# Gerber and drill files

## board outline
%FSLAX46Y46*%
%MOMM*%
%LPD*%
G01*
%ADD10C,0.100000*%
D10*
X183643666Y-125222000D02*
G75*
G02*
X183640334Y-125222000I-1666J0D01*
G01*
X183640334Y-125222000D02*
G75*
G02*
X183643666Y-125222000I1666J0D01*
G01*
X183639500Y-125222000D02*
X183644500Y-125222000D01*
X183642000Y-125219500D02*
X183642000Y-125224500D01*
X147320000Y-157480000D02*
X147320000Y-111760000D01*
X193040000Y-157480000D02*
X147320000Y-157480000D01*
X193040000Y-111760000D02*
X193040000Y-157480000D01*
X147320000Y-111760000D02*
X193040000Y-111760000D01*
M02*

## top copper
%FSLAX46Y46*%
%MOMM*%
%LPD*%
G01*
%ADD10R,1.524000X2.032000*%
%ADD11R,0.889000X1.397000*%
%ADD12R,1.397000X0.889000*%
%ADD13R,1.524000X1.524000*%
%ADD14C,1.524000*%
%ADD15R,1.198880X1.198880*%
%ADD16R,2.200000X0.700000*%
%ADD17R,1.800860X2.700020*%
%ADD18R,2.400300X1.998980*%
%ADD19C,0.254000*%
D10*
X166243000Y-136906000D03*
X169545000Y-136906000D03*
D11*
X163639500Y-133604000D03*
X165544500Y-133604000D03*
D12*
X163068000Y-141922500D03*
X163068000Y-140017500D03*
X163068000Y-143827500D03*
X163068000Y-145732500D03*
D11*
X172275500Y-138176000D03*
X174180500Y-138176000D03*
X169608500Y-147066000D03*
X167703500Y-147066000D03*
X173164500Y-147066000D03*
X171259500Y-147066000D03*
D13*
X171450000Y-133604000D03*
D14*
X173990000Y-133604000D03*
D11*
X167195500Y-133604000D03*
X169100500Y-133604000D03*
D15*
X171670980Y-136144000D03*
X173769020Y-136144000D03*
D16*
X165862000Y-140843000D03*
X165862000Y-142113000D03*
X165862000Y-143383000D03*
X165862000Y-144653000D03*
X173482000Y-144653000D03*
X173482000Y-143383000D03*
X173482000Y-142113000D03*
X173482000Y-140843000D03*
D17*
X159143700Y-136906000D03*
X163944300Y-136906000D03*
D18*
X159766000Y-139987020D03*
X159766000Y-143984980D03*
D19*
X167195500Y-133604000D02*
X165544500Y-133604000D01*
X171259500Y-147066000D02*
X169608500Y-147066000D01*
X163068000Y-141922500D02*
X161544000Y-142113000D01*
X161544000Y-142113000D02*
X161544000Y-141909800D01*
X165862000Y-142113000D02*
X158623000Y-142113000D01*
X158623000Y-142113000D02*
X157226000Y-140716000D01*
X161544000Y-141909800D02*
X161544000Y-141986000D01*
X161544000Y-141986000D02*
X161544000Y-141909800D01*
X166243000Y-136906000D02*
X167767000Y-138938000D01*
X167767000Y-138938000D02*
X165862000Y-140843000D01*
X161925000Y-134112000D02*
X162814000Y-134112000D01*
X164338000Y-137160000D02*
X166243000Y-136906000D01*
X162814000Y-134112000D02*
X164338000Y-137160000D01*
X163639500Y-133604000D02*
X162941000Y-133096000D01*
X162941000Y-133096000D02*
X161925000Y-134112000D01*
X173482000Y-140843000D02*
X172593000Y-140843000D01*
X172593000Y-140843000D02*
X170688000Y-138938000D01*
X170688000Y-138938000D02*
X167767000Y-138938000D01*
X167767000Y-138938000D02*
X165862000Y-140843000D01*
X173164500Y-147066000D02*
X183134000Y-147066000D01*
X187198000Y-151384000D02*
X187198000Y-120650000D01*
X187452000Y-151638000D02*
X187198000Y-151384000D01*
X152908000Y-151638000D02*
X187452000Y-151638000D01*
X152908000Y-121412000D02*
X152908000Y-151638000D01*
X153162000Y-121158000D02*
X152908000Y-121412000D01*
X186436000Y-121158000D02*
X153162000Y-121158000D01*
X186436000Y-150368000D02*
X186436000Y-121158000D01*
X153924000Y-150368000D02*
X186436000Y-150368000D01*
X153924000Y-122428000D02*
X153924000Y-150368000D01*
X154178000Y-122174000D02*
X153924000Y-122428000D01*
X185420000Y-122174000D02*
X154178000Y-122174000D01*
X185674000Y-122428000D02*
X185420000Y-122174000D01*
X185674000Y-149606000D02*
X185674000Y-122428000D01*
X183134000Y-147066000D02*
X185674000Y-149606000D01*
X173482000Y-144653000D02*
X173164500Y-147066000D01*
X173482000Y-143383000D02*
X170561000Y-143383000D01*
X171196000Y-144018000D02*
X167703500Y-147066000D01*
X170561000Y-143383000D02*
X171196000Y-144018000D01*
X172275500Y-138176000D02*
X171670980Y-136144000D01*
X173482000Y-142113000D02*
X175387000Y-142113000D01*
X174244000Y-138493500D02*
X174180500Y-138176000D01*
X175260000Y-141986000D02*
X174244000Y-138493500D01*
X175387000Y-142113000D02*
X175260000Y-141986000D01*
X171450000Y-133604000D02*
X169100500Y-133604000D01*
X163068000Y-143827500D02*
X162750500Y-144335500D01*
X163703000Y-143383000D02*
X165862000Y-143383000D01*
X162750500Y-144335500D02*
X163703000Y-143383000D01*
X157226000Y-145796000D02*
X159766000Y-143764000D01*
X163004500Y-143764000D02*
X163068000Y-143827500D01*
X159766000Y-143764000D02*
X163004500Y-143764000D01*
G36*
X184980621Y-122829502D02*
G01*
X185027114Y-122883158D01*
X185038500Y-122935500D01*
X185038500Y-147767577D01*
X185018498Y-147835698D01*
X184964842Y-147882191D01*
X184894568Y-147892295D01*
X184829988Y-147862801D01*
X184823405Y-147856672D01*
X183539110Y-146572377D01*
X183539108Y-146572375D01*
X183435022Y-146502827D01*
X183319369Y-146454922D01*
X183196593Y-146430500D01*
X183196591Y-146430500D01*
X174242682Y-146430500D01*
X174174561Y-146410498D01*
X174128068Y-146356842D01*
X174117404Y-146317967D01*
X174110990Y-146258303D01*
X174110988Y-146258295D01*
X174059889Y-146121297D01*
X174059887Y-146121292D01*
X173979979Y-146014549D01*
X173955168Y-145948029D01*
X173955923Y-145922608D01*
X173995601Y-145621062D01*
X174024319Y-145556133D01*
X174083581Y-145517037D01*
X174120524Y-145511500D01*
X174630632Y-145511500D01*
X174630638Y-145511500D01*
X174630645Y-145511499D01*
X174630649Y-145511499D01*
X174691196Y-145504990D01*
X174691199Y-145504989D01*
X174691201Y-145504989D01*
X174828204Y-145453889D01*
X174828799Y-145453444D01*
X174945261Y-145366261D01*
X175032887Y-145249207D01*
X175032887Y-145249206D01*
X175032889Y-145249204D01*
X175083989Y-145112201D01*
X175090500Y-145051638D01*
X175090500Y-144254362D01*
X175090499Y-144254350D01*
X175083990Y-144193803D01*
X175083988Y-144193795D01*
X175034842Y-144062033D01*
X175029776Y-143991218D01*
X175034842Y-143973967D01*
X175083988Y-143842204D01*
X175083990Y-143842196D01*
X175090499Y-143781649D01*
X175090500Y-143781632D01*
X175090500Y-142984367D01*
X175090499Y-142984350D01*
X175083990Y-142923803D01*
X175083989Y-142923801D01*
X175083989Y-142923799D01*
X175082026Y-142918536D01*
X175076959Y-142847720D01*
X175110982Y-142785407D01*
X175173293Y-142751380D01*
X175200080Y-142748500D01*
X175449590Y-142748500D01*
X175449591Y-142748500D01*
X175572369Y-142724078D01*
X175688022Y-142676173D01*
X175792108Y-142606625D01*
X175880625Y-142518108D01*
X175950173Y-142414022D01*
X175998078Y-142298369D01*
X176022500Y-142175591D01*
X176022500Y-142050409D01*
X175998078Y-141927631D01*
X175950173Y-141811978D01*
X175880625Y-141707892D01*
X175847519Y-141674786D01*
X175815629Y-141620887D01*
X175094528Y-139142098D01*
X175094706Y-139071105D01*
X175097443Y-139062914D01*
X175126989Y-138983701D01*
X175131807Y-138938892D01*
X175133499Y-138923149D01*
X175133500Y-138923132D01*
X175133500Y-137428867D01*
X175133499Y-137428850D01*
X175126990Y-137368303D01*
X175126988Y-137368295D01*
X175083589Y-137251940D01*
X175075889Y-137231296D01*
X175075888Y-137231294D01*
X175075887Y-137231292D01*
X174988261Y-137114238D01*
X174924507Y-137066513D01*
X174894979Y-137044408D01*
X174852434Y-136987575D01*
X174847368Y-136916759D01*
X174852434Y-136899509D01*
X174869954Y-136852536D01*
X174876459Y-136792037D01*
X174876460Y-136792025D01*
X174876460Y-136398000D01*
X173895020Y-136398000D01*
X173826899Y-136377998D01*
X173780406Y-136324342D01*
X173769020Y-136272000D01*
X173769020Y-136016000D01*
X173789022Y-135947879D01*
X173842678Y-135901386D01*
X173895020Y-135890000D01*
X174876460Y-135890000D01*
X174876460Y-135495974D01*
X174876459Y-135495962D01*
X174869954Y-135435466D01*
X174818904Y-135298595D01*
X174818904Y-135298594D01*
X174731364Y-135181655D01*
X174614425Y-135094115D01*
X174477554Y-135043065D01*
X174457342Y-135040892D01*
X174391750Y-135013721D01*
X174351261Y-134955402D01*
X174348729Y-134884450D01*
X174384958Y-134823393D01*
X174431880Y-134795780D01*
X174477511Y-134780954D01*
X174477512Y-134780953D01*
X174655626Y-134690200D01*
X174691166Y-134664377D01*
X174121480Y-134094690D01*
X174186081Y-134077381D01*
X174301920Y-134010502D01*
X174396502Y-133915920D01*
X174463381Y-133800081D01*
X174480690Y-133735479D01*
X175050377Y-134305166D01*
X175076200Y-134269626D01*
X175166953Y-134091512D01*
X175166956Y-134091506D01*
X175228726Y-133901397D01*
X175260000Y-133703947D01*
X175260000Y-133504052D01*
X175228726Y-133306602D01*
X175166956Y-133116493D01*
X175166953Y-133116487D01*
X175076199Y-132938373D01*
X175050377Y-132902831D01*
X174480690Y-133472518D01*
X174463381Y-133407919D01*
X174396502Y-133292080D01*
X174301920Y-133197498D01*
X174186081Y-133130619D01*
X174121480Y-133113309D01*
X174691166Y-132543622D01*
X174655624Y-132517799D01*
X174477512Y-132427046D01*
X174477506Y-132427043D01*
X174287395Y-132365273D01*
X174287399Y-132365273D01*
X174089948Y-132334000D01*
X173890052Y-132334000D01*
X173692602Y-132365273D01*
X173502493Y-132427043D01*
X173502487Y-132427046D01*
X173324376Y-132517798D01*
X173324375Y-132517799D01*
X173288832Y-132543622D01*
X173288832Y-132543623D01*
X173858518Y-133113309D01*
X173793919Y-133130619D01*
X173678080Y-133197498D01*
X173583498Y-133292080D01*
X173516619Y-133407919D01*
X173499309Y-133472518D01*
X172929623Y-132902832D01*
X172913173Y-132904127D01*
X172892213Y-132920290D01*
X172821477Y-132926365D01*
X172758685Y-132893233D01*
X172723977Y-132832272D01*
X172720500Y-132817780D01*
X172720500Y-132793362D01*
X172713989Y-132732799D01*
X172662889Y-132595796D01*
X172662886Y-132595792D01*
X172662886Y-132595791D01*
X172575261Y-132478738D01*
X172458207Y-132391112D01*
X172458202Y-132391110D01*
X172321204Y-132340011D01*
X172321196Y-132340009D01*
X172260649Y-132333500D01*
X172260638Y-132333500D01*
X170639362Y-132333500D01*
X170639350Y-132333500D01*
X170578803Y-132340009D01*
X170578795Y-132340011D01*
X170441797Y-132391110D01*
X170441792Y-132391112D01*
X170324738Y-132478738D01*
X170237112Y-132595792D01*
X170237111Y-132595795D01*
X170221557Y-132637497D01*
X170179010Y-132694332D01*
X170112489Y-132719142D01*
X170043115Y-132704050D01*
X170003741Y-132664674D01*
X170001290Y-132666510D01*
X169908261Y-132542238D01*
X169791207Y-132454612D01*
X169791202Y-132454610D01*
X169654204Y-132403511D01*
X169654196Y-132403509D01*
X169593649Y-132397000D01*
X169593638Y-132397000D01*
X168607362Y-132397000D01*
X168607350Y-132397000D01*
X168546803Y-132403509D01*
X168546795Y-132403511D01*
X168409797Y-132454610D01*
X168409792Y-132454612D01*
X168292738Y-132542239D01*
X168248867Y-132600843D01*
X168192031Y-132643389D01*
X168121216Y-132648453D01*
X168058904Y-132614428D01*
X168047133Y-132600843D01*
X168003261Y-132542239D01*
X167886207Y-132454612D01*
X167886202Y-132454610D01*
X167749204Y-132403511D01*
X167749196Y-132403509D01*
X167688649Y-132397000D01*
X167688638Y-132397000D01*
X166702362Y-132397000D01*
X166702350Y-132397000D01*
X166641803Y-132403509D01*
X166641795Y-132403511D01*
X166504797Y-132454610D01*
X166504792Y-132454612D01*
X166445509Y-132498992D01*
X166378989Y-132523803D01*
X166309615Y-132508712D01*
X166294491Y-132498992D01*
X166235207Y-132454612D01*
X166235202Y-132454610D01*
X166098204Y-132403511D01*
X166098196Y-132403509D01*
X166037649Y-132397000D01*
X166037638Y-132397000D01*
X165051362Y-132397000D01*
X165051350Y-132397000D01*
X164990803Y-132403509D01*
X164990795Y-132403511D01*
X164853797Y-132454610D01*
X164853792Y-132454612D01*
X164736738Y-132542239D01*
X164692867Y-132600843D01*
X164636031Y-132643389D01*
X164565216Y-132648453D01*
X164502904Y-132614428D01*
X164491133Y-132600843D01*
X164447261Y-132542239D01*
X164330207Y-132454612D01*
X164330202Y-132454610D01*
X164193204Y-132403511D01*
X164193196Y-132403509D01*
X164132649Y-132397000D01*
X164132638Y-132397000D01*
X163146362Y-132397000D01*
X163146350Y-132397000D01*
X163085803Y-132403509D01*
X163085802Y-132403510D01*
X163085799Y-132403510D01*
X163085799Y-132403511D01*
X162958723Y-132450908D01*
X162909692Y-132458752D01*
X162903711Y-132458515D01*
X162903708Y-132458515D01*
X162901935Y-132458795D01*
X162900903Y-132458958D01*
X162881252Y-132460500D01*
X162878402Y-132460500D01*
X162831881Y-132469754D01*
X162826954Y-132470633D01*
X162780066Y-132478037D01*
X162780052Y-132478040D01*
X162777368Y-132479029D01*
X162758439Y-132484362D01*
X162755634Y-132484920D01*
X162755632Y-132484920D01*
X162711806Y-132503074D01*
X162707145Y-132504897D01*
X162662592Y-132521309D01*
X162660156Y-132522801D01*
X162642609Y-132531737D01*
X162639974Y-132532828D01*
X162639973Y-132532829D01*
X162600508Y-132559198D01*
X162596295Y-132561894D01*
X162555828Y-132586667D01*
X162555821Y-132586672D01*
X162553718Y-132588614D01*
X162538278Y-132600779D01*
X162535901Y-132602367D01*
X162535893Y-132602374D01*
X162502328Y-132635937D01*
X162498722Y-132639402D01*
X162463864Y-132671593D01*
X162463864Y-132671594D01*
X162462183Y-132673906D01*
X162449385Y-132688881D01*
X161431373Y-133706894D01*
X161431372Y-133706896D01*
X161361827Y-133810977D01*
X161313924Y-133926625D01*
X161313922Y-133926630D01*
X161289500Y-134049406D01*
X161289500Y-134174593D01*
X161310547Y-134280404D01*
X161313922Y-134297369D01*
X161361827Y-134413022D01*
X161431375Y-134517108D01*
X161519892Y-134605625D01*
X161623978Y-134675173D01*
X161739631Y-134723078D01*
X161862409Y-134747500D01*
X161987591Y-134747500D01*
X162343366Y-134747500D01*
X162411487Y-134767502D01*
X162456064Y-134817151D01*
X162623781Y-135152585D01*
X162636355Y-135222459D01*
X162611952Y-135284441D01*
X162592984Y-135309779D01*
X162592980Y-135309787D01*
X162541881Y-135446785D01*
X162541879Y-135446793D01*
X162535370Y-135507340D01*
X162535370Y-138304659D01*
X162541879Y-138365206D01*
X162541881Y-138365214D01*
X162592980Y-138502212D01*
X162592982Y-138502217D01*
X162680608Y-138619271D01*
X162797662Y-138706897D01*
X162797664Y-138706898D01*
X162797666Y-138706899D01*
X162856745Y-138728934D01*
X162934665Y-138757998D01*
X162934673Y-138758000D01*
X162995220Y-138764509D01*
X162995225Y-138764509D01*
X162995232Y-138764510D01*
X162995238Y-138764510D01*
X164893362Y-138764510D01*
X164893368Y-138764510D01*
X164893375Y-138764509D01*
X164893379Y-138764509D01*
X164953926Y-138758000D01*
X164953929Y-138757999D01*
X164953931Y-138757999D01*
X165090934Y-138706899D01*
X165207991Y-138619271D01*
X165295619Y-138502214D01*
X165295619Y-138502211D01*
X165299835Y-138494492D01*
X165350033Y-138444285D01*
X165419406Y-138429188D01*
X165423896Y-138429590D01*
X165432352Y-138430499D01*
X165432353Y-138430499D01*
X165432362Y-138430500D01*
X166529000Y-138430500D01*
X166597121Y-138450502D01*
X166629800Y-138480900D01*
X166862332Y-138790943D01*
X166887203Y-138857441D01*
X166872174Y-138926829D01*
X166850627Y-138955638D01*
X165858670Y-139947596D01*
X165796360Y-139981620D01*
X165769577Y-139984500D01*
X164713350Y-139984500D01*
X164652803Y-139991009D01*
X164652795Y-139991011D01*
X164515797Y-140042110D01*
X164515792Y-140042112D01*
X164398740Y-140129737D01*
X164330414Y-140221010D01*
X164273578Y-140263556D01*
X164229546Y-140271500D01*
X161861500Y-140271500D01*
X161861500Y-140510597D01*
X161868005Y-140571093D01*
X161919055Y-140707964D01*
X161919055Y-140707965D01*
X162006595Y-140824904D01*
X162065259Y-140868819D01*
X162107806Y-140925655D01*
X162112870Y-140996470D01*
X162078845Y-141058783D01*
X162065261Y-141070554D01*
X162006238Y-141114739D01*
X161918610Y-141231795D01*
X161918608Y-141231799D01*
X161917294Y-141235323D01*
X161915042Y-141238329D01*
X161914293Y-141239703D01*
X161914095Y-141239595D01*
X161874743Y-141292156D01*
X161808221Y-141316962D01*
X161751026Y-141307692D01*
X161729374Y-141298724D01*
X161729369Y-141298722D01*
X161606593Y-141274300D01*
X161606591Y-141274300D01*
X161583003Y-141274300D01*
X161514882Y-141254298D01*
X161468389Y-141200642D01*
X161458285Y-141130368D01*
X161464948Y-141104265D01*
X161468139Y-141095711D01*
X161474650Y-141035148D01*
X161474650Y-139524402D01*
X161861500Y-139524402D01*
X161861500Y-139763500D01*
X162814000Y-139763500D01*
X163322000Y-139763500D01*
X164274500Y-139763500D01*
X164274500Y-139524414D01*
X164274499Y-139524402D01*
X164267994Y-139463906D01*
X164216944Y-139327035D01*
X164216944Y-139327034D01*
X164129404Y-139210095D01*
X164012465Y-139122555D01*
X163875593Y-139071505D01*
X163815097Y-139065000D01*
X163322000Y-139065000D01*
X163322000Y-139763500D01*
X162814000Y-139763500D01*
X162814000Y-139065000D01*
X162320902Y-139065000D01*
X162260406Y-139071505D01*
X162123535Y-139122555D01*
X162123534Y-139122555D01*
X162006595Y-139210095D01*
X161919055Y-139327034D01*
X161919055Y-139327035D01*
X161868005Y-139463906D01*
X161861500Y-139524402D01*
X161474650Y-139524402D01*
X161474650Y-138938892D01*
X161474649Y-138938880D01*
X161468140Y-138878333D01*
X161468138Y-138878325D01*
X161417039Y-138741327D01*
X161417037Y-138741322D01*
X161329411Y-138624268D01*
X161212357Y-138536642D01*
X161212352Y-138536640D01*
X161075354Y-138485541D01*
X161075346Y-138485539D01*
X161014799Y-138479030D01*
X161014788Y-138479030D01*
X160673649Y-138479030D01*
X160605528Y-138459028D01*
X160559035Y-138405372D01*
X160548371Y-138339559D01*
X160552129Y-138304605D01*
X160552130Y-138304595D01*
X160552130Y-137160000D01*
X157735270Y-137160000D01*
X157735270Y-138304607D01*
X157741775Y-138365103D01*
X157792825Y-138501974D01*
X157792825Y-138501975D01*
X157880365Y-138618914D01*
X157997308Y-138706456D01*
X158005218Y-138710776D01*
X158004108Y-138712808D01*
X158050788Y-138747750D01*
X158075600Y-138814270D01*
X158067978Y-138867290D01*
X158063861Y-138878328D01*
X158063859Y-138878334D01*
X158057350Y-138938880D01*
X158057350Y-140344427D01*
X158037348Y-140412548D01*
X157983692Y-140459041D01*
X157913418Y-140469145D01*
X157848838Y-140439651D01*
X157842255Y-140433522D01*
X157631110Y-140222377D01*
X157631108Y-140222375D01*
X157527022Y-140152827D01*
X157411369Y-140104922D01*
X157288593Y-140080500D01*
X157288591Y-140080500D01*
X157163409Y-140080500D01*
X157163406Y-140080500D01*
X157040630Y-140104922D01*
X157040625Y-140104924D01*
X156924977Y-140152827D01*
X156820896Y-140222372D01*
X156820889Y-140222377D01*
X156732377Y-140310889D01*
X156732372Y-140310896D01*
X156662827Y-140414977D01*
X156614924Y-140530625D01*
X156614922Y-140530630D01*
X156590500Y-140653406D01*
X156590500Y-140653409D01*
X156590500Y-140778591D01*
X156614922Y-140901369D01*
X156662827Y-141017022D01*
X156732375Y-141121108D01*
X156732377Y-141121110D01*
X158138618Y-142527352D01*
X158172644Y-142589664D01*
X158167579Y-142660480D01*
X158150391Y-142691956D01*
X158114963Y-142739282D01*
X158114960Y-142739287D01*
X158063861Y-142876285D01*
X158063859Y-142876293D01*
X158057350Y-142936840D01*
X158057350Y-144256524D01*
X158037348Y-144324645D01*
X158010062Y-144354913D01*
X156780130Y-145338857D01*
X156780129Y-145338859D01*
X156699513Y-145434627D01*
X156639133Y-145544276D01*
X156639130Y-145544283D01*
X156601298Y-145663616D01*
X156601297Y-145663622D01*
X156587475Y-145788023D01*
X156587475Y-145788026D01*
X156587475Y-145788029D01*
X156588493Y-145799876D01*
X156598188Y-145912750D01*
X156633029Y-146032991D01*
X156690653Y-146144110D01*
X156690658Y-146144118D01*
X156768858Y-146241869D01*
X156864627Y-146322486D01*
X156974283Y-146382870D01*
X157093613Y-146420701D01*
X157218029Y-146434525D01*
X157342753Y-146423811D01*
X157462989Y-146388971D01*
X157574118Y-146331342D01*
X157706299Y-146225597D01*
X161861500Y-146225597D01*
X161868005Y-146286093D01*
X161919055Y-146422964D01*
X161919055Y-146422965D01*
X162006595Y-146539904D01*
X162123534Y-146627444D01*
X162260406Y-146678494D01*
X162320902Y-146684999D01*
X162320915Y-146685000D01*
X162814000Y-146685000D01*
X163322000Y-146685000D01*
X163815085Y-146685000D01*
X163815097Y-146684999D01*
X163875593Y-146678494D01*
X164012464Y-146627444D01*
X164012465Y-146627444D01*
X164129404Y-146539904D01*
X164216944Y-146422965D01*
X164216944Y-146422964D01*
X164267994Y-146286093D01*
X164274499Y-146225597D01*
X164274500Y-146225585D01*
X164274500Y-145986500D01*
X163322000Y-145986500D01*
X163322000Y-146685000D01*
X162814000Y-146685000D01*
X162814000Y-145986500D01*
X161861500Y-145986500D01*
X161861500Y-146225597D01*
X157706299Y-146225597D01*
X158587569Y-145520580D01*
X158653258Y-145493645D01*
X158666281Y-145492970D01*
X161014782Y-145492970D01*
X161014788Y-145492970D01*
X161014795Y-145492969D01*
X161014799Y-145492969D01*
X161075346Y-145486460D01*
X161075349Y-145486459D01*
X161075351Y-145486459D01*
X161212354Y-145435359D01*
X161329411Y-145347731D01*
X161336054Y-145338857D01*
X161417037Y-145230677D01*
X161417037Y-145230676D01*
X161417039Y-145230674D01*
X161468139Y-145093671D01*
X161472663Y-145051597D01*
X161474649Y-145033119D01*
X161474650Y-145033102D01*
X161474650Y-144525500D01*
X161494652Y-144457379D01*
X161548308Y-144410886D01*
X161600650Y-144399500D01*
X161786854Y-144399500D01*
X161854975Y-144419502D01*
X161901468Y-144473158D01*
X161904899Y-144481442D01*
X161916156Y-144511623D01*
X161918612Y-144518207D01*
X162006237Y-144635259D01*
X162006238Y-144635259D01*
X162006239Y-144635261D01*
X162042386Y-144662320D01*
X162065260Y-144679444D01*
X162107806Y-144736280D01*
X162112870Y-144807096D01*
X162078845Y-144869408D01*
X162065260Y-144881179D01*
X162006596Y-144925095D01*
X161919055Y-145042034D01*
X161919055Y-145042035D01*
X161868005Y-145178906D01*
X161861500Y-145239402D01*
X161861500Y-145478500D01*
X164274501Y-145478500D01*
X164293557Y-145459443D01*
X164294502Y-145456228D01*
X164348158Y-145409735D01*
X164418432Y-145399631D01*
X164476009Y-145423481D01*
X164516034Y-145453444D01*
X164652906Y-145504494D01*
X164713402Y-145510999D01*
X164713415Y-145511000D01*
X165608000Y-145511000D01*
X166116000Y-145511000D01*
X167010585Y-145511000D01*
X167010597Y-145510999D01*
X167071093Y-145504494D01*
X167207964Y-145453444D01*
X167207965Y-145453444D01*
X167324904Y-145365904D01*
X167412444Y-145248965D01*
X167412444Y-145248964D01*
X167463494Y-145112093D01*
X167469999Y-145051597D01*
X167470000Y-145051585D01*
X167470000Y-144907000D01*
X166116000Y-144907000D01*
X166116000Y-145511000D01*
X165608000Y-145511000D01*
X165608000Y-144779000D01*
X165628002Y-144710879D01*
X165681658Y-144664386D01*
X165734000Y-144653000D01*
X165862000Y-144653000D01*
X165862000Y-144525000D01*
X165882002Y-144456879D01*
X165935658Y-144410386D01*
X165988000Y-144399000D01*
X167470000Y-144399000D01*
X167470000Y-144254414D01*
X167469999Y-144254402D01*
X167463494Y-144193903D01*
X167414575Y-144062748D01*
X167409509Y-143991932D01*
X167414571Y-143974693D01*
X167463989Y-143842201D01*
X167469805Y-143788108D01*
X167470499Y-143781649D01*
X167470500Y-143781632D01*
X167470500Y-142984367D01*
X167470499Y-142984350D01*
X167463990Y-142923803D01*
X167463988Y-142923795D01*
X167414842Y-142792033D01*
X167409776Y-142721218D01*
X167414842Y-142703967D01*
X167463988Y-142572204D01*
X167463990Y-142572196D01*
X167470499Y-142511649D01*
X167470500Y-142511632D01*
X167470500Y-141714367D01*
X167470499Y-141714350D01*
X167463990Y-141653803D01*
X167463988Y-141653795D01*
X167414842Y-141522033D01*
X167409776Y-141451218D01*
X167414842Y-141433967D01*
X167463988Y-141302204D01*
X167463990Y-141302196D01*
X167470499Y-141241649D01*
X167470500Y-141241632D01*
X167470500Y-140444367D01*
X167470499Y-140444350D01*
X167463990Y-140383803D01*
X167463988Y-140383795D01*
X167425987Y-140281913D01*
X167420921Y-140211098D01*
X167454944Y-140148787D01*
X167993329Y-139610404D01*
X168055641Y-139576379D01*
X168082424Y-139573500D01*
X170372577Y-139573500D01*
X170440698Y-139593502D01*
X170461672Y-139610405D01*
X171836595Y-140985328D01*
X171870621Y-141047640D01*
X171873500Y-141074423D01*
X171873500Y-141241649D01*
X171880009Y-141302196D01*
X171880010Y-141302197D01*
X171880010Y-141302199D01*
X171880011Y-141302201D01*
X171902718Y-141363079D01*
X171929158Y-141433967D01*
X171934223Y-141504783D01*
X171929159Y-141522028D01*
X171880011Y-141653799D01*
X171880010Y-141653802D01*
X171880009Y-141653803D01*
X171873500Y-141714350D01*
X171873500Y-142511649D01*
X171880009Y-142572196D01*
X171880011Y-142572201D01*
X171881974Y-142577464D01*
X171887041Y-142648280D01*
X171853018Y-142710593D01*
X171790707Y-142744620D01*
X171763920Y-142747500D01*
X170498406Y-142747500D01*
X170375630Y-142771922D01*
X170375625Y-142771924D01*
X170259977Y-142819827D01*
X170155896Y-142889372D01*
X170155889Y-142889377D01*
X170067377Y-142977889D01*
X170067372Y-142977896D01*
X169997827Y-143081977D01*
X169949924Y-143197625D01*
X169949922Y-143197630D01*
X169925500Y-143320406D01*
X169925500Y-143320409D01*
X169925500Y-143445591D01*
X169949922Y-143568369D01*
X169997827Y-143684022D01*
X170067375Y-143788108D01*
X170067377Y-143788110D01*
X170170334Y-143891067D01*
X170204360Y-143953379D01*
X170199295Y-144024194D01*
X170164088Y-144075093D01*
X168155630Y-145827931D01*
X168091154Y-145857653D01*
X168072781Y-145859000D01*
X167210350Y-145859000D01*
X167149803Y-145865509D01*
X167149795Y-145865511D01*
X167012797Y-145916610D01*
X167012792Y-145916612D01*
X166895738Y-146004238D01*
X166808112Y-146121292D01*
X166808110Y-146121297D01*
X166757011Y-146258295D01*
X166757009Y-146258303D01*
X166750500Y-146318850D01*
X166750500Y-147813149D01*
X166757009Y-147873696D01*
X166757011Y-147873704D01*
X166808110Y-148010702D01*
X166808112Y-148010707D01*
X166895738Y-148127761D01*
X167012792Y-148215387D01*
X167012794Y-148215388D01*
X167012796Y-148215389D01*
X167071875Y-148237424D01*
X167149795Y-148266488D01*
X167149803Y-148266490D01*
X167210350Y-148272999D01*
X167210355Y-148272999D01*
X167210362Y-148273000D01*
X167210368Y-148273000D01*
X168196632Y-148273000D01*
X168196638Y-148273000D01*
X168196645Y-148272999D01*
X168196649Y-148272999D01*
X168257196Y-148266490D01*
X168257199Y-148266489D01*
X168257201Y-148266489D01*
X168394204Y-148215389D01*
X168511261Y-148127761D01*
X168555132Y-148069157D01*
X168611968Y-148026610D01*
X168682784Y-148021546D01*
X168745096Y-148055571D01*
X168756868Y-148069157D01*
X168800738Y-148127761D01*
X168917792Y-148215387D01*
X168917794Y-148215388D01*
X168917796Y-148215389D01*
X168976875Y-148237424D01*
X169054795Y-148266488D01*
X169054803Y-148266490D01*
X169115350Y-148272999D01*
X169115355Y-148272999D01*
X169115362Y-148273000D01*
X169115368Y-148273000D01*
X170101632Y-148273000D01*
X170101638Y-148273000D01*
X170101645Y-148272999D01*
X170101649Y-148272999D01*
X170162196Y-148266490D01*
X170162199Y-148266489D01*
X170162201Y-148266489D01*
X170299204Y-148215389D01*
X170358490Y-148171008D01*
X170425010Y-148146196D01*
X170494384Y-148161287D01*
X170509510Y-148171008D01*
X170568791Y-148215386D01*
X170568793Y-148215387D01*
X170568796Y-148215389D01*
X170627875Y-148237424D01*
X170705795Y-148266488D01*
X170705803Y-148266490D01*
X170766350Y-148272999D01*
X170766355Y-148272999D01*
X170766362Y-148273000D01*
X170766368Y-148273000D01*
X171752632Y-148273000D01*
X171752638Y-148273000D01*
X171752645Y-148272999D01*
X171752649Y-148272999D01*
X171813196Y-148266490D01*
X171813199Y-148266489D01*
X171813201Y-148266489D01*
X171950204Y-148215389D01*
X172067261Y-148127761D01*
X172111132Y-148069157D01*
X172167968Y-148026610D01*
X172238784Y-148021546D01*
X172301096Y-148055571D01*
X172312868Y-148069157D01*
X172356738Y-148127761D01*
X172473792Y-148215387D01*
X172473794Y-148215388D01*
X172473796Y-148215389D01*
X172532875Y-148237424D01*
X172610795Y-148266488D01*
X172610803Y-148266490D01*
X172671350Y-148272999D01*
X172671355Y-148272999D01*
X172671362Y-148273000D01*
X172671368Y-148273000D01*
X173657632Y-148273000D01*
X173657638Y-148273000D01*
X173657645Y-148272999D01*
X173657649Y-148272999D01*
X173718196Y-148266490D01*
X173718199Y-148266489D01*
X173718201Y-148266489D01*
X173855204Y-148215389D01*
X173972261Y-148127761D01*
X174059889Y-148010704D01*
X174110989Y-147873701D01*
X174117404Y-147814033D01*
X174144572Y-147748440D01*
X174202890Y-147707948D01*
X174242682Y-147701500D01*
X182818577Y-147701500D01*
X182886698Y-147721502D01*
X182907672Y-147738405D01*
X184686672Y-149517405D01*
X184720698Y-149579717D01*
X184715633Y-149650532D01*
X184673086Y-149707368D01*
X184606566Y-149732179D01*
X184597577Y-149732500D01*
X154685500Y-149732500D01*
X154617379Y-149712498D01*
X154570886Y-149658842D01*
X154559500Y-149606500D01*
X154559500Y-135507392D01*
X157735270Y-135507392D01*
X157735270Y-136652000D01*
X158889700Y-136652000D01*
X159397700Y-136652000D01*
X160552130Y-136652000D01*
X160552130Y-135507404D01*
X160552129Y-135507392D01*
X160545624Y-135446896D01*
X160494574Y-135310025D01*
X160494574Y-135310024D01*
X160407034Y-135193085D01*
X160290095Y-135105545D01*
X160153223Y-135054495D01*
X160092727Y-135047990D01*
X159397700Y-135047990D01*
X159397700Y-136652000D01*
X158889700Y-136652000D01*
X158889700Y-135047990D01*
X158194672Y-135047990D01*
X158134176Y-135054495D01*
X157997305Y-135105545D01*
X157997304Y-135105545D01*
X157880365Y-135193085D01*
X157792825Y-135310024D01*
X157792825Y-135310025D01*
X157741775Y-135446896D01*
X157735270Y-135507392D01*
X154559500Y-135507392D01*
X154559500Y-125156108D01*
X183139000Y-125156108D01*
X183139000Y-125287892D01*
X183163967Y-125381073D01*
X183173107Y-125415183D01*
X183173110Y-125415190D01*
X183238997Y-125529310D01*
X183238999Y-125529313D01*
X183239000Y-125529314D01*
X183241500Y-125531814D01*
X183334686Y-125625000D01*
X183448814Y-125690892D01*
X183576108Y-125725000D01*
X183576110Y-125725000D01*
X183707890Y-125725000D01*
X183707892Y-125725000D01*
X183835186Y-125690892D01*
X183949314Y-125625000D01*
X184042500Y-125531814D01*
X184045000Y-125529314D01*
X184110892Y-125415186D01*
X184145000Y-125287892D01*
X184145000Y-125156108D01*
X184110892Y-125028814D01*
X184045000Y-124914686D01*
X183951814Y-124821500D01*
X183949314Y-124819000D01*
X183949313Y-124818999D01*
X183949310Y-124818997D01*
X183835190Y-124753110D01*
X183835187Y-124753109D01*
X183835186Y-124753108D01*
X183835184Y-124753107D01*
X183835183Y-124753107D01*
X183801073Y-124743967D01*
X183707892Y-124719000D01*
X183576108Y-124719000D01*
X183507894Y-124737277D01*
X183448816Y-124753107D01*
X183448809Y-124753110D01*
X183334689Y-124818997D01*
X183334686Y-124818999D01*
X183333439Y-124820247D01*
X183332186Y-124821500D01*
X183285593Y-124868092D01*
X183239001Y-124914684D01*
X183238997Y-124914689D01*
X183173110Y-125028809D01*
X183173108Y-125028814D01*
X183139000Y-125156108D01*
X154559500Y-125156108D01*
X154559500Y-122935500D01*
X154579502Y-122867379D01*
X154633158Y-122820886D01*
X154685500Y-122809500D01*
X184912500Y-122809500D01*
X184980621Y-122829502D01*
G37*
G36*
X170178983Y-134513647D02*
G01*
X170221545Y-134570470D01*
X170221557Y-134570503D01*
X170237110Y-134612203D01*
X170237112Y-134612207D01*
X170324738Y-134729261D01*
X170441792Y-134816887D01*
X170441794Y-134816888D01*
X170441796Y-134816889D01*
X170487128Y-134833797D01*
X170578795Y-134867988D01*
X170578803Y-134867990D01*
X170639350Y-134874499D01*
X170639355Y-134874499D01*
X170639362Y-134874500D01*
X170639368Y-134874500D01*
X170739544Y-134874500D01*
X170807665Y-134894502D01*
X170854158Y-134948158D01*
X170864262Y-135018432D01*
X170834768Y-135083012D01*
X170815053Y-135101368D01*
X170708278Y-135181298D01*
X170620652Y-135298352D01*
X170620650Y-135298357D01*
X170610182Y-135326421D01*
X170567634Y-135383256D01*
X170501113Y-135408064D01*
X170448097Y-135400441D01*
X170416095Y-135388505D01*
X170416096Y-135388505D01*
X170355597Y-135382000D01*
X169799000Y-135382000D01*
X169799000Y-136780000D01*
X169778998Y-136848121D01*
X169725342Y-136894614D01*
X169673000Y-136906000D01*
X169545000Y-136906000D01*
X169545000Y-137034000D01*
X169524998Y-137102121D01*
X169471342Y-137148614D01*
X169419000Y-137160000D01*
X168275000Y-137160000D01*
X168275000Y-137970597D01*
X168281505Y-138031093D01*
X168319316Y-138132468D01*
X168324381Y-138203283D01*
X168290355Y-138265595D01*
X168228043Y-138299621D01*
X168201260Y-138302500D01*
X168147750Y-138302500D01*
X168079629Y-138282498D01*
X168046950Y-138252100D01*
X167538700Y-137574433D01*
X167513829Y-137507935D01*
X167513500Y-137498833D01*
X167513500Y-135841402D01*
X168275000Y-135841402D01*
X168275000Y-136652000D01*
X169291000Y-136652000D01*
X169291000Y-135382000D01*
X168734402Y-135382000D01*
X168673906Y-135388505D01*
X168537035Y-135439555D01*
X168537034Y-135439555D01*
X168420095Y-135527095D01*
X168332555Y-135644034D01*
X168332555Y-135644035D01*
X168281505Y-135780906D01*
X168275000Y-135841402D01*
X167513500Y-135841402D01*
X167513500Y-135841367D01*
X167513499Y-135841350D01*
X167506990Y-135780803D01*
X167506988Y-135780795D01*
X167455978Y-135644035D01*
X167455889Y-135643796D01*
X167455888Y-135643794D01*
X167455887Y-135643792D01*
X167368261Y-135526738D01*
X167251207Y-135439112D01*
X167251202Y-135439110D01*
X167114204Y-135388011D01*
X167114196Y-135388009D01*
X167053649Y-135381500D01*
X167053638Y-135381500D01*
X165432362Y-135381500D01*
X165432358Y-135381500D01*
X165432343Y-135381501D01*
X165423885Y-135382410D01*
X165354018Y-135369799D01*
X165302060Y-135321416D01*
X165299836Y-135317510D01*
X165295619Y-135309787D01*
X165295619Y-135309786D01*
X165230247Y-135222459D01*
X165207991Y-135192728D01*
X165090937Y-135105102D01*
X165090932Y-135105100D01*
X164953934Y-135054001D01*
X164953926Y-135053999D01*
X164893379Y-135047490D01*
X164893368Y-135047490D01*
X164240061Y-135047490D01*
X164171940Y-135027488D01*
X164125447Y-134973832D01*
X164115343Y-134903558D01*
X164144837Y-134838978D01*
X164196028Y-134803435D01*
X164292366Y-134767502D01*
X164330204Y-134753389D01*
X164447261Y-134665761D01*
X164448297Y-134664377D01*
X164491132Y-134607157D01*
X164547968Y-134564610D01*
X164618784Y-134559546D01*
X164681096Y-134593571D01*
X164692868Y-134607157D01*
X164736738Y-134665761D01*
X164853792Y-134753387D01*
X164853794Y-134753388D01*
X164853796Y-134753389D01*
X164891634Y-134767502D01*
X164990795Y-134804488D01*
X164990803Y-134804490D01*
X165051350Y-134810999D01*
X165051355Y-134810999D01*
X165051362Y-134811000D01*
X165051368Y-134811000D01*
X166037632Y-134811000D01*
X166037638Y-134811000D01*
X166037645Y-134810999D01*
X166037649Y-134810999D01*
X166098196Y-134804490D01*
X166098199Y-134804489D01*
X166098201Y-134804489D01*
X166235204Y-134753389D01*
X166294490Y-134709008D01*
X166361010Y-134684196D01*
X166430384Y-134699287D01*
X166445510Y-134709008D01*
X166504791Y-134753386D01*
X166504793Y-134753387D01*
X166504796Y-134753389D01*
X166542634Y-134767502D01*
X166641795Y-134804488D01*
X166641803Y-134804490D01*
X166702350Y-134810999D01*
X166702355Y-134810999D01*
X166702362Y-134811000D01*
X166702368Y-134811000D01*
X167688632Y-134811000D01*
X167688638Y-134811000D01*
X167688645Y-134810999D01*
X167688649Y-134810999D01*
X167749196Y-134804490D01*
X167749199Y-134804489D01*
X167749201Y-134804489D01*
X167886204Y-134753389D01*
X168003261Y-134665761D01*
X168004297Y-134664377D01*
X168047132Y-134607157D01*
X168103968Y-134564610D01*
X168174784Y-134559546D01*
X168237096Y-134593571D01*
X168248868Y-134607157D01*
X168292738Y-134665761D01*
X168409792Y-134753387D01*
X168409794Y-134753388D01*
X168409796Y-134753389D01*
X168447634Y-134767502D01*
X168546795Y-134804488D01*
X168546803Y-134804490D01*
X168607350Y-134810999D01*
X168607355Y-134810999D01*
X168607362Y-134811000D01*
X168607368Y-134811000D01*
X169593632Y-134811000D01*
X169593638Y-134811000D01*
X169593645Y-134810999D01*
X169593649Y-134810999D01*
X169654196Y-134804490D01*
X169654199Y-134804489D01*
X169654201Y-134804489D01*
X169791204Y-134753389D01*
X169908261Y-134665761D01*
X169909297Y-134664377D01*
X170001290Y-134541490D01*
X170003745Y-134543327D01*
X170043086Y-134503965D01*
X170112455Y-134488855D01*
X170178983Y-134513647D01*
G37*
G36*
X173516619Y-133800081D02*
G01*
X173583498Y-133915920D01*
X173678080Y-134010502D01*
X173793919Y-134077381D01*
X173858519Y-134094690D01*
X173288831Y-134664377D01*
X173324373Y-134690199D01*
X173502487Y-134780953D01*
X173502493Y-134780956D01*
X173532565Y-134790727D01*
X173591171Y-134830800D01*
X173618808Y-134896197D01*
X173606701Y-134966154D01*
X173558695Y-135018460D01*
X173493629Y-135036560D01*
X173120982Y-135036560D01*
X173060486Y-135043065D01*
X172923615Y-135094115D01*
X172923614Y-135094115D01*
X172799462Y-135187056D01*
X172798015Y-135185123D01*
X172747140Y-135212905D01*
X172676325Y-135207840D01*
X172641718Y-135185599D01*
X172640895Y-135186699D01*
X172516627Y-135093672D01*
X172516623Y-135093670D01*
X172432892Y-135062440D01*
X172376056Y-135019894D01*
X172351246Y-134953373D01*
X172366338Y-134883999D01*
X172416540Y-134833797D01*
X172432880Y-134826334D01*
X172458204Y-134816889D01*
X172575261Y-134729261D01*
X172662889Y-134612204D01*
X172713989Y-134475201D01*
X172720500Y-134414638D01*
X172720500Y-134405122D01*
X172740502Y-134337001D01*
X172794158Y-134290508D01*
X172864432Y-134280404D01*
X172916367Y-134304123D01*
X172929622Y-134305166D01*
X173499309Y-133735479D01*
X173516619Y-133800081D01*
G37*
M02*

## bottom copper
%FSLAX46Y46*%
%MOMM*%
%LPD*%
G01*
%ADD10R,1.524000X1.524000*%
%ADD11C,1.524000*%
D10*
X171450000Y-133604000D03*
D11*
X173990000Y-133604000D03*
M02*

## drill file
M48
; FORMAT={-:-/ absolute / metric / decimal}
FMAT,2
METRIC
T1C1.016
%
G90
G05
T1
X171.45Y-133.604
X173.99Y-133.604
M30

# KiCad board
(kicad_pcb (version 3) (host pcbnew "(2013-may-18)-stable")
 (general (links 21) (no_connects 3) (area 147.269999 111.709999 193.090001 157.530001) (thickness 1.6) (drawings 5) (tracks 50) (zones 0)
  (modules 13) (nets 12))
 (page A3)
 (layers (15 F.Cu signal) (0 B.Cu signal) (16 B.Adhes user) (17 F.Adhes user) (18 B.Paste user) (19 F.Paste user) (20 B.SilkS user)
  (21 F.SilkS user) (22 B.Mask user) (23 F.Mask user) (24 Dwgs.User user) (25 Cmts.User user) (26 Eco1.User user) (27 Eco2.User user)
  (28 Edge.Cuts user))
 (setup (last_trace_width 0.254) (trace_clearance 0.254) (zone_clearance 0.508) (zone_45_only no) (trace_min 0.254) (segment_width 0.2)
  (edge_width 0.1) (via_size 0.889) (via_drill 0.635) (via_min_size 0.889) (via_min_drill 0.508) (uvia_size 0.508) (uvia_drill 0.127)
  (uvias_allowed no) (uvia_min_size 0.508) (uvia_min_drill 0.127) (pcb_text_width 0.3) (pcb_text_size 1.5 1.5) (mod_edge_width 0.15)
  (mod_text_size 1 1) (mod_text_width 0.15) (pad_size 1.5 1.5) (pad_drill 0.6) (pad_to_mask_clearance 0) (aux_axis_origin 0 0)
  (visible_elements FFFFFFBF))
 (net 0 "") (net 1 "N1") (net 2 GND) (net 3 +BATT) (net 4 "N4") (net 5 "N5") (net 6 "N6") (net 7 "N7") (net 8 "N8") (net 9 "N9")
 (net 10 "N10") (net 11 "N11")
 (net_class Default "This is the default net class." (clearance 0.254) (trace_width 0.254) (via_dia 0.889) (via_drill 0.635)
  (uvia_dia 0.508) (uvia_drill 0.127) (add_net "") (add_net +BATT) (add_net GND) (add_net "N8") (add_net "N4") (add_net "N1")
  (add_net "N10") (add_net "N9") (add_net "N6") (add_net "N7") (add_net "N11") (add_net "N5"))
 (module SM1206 (layer F.Cu) (at 167.894 136.906)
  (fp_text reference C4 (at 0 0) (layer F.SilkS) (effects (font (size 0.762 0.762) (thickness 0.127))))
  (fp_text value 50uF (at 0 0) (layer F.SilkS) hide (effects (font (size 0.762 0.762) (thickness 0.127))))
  (pad 1 smd rect (at -1.651 0) (size 1.524 2.032) (layers F.Cu F.Paste F.Mask) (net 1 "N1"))
  (pad 2 smd rect (at 1.651 0) (size 1.524 2.032) (layers F.Cu F.Paste F.Mask) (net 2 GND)))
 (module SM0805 (layer F.Cu) (at 164.592 133.604)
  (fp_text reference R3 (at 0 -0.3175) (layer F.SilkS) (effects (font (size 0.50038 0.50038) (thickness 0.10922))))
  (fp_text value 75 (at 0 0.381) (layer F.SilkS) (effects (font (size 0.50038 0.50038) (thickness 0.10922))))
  (pad 1 smd rect (at -0.9525 0) (size 0.889 1.397) (layers F.Cu F.Paste F.Mask) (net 1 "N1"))
  (pad 2 smd rect (at 0.9525 0) (size 0.889 1.397) (layers F.Cu F.Paste F.Mask) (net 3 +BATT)))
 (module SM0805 (layer F.Cu) (at 163.068 140.97 90)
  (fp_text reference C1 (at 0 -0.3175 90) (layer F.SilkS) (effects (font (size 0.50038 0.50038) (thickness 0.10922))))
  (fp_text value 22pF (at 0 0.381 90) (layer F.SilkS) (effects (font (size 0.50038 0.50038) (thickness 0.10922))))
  (pad 1 smd rect (at -0.9525 0 90) (size 0.889 1.397) (layers F.Cu F.Paste F.Mask) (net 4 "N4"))
  (pad 2 smd rect (at 0.9525 0 90) (size 0.889 1.397) (layers F.Cu F.Paste F.Mask) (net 2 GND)))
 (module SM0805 (layer F.Cu) (at 163.068 144.78 270)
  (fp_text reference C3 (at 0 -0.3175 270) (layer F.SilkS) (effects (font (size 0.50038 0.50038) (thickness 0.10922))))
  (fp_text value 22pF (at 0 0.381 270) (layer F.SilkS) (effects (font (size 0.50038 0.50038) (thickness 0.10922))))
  (pad 1 smd rect (at -0.9525 0 270) (size 0.889 1.397) (layers F.Cu F.Paste F.Mask) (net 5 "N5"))
  (pad 2 smd rect (at 0.9525 0 270) (size 0.889 1.397) (layers F.Cu F.Paste F.Mask) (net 2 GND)))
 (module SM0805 (layer F.Cu) (at 173.228 138.176)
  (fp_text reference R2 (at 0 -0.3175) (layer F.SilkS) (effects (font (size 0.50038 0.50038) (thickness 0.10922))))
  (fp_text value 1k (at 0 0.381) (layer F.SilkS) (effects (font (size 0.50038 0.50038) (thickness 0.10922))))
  (pad 1 smd rect (at -0.9525 0) (size 0.889 1.397) (layers F.Cu F.Paste F.Mask) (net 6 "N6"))
  (pad 2 smd rect (at 0.9525 0) (size 0.889 1.397) (layers F.Cu F.Paste F.Mask) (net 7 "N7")))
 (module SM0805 (layer F.Cu) (at 168.656 147.066 180)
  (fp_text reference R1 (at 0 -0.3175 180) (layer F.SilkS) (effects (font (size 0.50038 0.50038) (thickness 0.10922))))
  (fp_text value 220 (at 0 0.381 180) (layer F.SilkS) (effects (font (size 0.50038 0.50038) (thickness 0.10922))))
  (pad 1 smd rect (at -0.9525 0 180) (size 0.889 1.397) (layers F.Cu F.Paste F.Mask) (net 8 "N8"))
  (pad 2 smd rect (at 0.9525 0 180) (size 0.889 1.397) (layers F.Cu F.Paste F.Mask) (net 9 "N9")))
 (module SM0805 (layer F.Cu) (at 172.212 147.066 180)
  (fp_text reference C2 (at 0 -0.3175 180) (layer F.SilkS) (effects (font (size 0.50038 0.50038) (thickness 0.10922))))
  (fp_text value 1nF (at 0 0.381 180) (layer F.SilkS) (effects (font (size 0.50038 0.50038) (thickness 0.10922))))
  (pad 1 smd rect (at -0.9525 0 180) (size 0.889 1.397) (layers F.Cu F.Paste F.Mask) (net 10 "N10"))
  (pad 2 smd rect (at 0.9525 0 180) (size 0.889 1.397) (layers F.Cu F.Paste F.Mask) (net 8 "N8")))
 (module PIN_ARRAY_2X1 (layer F.Cu) (at 172.72 133.604)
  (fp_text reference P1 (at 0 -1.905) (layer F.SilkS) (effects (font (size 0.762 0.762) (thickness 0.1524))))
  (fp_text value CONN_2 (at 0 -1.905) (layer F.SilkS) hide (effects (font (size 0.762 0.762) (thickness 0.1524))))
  (pad 1 thru_hole rect (at -1.27 0) (size 1.524 1.524) (drill 1.016) (layers *.Cu *.Mask F.SilkS) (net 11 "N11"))
  (pad 2 thru_hole circle (at 1.27 0) (size 1.524 1.524) (drill 1.016) (layers *.Cu *.Mask F.SilkS) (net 2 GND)))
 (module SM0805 (layer F.Cu) (at 168.148 133.604)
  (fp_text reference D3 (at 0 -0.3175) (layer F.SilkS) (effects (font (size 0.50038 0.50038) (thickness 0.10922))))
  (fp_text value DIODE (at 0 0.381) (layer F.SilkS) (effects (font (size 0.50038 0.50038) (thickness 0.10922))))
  (pad 1 smd rect (at -0.9525 0) (size 0.889 1.397) (layers F.Cu F.Paste F.Mask) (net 3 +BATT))
  (pad 2 smd rect (at 0.9525 0) (size 0.889 1.397) (layers F.Cu F.Paste F.Mask) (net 11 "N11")))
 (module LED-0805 (layer F.Cu) (at 172.72 136.144)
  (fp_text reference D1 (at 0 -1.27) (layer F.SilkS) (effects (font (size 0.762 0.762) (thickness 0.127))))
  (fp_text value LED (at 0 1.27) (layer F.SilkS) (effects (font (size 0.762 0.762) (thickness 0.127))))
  (pad 1 smd rect (at -1.04902 0) (size 1.19888 1.19888) (layers F.Cu F.Paste F.Mask) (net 6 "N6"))
  (pad 2 smd rect (at 1.04902 0) (size 1.19888 1.19888) (layers F.Cu F.Paste F.Mask) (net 2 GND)))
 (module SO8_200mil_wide (layer F.Cu) (at 169.672 142.748 270)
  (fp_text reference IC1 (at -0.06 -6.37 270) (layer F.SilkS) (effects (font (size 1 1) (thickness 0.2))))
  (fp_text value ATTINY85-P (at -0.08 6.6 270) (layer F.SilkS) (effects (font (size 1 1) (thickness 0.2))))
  (pad 1 smd rect (at -1.905 3.81 270) (size 0.7 2.2) (layers F.Cu F.Paste F.Mask) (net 1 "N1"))
  (pad 2 smd rect (at -0.635 3.81 270) (size 0.7 2.2) (layers F.Cu F.Paste F.Mask) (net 4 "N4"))
  (pad 3 smd rect (at 0.635 3.81 270) (size 0.7 2.2) (layers F.Cu F.Paste F.Mask) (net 5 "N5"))
  (pad 4 smd rect (at 1.905 3.81 270) (size 0.7 2.2) (layers F.Cu F.Paste F.Mask) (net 2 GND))
  (pad 5 smd rect (at 1.905 -3.81 270) (size 0.7 2.2) (layers F.Cu F.Paste F.Mask) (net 10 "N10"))
  (pad 6 smd rect (at 0.635 -3.81 270) (size 0.7 2.2) (layers F.Cu F.Paste F.Mask) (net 9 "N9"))
  (pad 7 smd rect (at -0.635 -3.81 270) (size 0.7 2.2) (layers F.Cu F.Paste F.Mask) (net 7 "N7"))
  (pad 8 smd rect (at -1.905 -3.81 270) (size 0.7 2.2) (layers F.Cu F.Paste F.Mask) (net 1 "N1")))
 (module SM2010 (layer F.Cu) (at 161.544 136.906)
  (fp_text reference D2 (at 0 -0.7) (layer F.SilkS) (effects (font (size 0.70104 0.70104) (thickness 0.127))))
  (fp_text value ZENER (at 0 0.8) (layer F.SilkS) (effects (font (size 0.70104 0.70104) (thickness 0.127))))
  (pad 1 smd rect (at -2.4003 0) (size 1.80086 2.70002) (layers F.Cu F.Paste F.Mask) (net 2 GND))
  (pad 2 smd rect (at 2.4003 0) (size 1.80086 2.70002) (layers F.Cu F.Paste F.Mask) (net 1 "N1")))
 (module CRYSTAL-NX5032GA (layer F.Cu) (at 159.766 141.986 270)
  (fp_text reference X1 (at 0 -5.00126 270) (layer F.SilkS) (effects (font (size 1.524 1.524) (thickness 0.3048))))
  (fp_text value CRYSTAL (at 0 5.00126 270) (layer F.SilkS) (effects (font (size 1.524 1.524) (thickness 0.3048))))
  (pad 1 smd rect (at -1.99898 0 270) (size 1.99898 2.4003) (layers F.Cu F.Paste F.Mask) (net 4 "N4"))
  (pad 2 smd rect (at 1.99898 0 270) (size 1.99898 2.4003) (layers F.Cu F.Paste F.Mask) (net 5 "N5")))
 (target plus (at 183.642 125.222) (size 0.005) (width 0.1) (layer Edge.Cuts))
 (gr_line (start 147.32 157.48) (end 147.32 111.76) (angle 90) (layer Edge.Cuts) (width 0.1))
 (gr_line (start 193.04 157.48) (end 147.32 157.48) (angle 90) (layer Edge.Cuts) (width 0.1))
 (gr_line (start 193.04 111.76) (end 193.04 157.48) (angle 90) (layer Edge.Cuts) (width 0.1))
 (gr_line (start 147.32 111.76) (end 193.04 111.76) (angle 90) (layer Edge.Cuts) (width 0.1))
 (segment (start 167.1955 133.604) (end 165.5445 133.604) (width 0.254) (layer F.Cu) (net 3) (status 10))
 (segment (start 171.2595 147.066) (end 169.6085 147.066) (width 0.254) (layer F.Cu) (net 8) (status 10))
 (segment (start 163.068 141.9225) (end 161.544 142.113) (width 0.254) (layer F.Cu) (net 4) (status 10))
 (segment (start 161.544 142.113) (end 161.544 141.9098) (width 0.254) (layer F.Cu) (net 4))
 (segment (start 165.862 142.113) (end 158.623 142.113) (width 0.254) (layer F.Cu) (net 4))
 (segment (start 158.623 142.113) (end 157.226 140.716) (width 0.254) (layer F.Cu) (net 4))
 (segment (start 161.544 141.9098) (end 161.544 141.986) (width 0.254) (layer F.Cu) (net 4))
 (segment (start 161.544 141.986) (end 161.544 141.9098) (width 0.254) (layer F.Cu) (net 4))
 (segment (start 166.243 136.906) (end 167.767 138.938) (width 0.254) (layer F.Cu) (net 1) (status 10))
 (segment (start 167.767 138.938) (end 165.862 140.843) (width 0.254) (layer F.Cu) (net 1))
 (segment (start 161.925 134.112) (end 162.814 134.112) (width 0.254) (layer F.Cu) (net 1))
 (segment (start 164.338 137.16) (end 166.243 136.906) (width 0.254) (layer F.Cu) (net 1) (status 20))
 (segment (start 162.814 134.112) (end 164.338 137.16) (width 0.254) (layer F.Cu) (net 1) (status 20))
 (segment (start 163.6395 133.604) (end 162.941 133.096) (width 0.254) (layer F.Cu) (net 1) (status 10))
 (segment (start 162.941 133.096) (end 161.925 134.112) (width 0.254) (layer F.Cu) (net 1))
 (segment (start 173.482 140.843) (end 172.593 140.843) (width 0.254) (layer F.Cu) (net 1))
 (segment (start 172.593 140.843) (end 170.688 138.938) (width 0.254) (layer F.Cu) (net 1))
 (segment (start 170.688 138.938) (end 167.767 138.938) (width 0.254) (layer F.Cu) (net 1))
 (segment (start 167.767 138.938) (end 165.862 140.843) (width 0.254) (layer F.Cu) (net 1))
 (segment (start 173.1645 147.066) (end 183.134 147.066) (width 0.254) (layer F.Cu) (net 10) (status 400000))
 (segment (start 187.198 151.384) (end 187.198 120.65) (width 0.254) (layer F.Cu) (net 10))
 (segment (start 187.452 151.638) (end 187.198 151.384) (width 0.254) (layer F.Cu) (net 10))
 (segment (start 152.908 151.638) (end 187.452 151.638) (width 0.254) (layer F.Cu) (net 10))
 (segment (start 152.908 121.412) (end 152.908 151.638) (width 0.254) (layer F.Cu) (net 10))
 (segment (start 153.162 121.158) (end 152.908 121.412) (width 0.254) (layer F.Cu) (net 10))
 (segment (start 186.436 121.158) (end 153.162 121.158) (width 0.254) (layer F.Cu) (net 10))
 (segment (start 186.436 150.368) (end 186.436 121.158) (width 0.254) (layer F.Cu) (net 10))
 (segment (start 153.924 150.368) (end 186.436 150.368) (width 0.254) (layer F.Cu) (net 10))
 (segment (start 153.924 122.428) (end 153.924 150.368) (width 0.254) (layer F.Cu) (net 10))
 (segment (start 154.178 122.174) (end 153.924 122.428) (width 0.254) (layer F.Cu) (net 10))
 (segment (start 185.42 122.174) (end 154.178 122.174) (width 0.254) (layer F.Cu) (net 10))
 (segment (start 185.674 122.428) (end 185.42 122.174) (width 0.254) (layer F.Cu) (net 10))
 (segment (start 185.674 149.606) (end 185.674 122.428) (width 0.254) (layer F.Cu) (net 10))
 (segment (start 183.134 147.066) (end 185.674 149.606) (width 0.254) (layer F.Cu) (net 10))
 (segment (start 173.482 144.653) (end 173.1645 147.066) (width 0.254) (layer F.Cu) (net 10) (status 20))
 (segment (start 173.482 143.383) (end 170.561 143.383) (width 0.254) (layer F.Cu) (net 9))
 (segment (start 171.196 144.018) (end 167.7035 147.066) (width 0.254) (layer F.Cu) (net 9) (status 20))
 (segment (start 170.561 143.383) (end 171.196 144.018) (width 0.254) (layer F.Cu) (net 9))
 (segment (start 172.2755 138.176) (end 171.67098 136.144) (width 0.254) (layer F.Cu) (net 6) (status 10))
 (segment (start 173.482 142.113) (end 175.387 142.113) (width 0.254) (layer F.Cu) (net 7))
 (segment (start 174.244 138.4935) (end 174.1805 138.176) (width 0.254) (layer F.Cu) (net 7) (status 30))
 (segment (start 175.26 141.986) (end 174.244 138.4935) (width 0.254) (layer F.Cu) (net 7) (status 20))
 (segment (start 175.387 142.113) (end 175.26 141.986) (width 0.254) (layer F.Cu) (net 7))
 (segment (start 171.45 133.604) (end 169.1005 133.604) (width 0.254) (layer F.Cu) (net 11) (status 10))
 (segment (start 163.068 143.8275) (end 162.7505 144.3355) (width 0.254) (layer F.Cu) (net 5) (status 10))
 (segment (start 163.703 143.383) (end 165.862 143.383) (width 0.254) (layer F.Cu) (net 5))
 (segment (start 162.7505 144.3355) (end 163.703 143.383) (width 0.254) (layer F.Cu) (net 5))
 (segment (start 157.226 145.796) (end 159.766 143.764) (width 0.254) (layer F.Cu) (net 5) (status 20))
 (segment (start 163.0045 143.764) (end 163.068 143.8275) (width 0.254) (layer F.Cu) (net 5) (status 30))
 (segment (start 159.766 143.764) (end 163.0045 143.764) (width 0.254) (layer F.Cu) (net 5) (status 10))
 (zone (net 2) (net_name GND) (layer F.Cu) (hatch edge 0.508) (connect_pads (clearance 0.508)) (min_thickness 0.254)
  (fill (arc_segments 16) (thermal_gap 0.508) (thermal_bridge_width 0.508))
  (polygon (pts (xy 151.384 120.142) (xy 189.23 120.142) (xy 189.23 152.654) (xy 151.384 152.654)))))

